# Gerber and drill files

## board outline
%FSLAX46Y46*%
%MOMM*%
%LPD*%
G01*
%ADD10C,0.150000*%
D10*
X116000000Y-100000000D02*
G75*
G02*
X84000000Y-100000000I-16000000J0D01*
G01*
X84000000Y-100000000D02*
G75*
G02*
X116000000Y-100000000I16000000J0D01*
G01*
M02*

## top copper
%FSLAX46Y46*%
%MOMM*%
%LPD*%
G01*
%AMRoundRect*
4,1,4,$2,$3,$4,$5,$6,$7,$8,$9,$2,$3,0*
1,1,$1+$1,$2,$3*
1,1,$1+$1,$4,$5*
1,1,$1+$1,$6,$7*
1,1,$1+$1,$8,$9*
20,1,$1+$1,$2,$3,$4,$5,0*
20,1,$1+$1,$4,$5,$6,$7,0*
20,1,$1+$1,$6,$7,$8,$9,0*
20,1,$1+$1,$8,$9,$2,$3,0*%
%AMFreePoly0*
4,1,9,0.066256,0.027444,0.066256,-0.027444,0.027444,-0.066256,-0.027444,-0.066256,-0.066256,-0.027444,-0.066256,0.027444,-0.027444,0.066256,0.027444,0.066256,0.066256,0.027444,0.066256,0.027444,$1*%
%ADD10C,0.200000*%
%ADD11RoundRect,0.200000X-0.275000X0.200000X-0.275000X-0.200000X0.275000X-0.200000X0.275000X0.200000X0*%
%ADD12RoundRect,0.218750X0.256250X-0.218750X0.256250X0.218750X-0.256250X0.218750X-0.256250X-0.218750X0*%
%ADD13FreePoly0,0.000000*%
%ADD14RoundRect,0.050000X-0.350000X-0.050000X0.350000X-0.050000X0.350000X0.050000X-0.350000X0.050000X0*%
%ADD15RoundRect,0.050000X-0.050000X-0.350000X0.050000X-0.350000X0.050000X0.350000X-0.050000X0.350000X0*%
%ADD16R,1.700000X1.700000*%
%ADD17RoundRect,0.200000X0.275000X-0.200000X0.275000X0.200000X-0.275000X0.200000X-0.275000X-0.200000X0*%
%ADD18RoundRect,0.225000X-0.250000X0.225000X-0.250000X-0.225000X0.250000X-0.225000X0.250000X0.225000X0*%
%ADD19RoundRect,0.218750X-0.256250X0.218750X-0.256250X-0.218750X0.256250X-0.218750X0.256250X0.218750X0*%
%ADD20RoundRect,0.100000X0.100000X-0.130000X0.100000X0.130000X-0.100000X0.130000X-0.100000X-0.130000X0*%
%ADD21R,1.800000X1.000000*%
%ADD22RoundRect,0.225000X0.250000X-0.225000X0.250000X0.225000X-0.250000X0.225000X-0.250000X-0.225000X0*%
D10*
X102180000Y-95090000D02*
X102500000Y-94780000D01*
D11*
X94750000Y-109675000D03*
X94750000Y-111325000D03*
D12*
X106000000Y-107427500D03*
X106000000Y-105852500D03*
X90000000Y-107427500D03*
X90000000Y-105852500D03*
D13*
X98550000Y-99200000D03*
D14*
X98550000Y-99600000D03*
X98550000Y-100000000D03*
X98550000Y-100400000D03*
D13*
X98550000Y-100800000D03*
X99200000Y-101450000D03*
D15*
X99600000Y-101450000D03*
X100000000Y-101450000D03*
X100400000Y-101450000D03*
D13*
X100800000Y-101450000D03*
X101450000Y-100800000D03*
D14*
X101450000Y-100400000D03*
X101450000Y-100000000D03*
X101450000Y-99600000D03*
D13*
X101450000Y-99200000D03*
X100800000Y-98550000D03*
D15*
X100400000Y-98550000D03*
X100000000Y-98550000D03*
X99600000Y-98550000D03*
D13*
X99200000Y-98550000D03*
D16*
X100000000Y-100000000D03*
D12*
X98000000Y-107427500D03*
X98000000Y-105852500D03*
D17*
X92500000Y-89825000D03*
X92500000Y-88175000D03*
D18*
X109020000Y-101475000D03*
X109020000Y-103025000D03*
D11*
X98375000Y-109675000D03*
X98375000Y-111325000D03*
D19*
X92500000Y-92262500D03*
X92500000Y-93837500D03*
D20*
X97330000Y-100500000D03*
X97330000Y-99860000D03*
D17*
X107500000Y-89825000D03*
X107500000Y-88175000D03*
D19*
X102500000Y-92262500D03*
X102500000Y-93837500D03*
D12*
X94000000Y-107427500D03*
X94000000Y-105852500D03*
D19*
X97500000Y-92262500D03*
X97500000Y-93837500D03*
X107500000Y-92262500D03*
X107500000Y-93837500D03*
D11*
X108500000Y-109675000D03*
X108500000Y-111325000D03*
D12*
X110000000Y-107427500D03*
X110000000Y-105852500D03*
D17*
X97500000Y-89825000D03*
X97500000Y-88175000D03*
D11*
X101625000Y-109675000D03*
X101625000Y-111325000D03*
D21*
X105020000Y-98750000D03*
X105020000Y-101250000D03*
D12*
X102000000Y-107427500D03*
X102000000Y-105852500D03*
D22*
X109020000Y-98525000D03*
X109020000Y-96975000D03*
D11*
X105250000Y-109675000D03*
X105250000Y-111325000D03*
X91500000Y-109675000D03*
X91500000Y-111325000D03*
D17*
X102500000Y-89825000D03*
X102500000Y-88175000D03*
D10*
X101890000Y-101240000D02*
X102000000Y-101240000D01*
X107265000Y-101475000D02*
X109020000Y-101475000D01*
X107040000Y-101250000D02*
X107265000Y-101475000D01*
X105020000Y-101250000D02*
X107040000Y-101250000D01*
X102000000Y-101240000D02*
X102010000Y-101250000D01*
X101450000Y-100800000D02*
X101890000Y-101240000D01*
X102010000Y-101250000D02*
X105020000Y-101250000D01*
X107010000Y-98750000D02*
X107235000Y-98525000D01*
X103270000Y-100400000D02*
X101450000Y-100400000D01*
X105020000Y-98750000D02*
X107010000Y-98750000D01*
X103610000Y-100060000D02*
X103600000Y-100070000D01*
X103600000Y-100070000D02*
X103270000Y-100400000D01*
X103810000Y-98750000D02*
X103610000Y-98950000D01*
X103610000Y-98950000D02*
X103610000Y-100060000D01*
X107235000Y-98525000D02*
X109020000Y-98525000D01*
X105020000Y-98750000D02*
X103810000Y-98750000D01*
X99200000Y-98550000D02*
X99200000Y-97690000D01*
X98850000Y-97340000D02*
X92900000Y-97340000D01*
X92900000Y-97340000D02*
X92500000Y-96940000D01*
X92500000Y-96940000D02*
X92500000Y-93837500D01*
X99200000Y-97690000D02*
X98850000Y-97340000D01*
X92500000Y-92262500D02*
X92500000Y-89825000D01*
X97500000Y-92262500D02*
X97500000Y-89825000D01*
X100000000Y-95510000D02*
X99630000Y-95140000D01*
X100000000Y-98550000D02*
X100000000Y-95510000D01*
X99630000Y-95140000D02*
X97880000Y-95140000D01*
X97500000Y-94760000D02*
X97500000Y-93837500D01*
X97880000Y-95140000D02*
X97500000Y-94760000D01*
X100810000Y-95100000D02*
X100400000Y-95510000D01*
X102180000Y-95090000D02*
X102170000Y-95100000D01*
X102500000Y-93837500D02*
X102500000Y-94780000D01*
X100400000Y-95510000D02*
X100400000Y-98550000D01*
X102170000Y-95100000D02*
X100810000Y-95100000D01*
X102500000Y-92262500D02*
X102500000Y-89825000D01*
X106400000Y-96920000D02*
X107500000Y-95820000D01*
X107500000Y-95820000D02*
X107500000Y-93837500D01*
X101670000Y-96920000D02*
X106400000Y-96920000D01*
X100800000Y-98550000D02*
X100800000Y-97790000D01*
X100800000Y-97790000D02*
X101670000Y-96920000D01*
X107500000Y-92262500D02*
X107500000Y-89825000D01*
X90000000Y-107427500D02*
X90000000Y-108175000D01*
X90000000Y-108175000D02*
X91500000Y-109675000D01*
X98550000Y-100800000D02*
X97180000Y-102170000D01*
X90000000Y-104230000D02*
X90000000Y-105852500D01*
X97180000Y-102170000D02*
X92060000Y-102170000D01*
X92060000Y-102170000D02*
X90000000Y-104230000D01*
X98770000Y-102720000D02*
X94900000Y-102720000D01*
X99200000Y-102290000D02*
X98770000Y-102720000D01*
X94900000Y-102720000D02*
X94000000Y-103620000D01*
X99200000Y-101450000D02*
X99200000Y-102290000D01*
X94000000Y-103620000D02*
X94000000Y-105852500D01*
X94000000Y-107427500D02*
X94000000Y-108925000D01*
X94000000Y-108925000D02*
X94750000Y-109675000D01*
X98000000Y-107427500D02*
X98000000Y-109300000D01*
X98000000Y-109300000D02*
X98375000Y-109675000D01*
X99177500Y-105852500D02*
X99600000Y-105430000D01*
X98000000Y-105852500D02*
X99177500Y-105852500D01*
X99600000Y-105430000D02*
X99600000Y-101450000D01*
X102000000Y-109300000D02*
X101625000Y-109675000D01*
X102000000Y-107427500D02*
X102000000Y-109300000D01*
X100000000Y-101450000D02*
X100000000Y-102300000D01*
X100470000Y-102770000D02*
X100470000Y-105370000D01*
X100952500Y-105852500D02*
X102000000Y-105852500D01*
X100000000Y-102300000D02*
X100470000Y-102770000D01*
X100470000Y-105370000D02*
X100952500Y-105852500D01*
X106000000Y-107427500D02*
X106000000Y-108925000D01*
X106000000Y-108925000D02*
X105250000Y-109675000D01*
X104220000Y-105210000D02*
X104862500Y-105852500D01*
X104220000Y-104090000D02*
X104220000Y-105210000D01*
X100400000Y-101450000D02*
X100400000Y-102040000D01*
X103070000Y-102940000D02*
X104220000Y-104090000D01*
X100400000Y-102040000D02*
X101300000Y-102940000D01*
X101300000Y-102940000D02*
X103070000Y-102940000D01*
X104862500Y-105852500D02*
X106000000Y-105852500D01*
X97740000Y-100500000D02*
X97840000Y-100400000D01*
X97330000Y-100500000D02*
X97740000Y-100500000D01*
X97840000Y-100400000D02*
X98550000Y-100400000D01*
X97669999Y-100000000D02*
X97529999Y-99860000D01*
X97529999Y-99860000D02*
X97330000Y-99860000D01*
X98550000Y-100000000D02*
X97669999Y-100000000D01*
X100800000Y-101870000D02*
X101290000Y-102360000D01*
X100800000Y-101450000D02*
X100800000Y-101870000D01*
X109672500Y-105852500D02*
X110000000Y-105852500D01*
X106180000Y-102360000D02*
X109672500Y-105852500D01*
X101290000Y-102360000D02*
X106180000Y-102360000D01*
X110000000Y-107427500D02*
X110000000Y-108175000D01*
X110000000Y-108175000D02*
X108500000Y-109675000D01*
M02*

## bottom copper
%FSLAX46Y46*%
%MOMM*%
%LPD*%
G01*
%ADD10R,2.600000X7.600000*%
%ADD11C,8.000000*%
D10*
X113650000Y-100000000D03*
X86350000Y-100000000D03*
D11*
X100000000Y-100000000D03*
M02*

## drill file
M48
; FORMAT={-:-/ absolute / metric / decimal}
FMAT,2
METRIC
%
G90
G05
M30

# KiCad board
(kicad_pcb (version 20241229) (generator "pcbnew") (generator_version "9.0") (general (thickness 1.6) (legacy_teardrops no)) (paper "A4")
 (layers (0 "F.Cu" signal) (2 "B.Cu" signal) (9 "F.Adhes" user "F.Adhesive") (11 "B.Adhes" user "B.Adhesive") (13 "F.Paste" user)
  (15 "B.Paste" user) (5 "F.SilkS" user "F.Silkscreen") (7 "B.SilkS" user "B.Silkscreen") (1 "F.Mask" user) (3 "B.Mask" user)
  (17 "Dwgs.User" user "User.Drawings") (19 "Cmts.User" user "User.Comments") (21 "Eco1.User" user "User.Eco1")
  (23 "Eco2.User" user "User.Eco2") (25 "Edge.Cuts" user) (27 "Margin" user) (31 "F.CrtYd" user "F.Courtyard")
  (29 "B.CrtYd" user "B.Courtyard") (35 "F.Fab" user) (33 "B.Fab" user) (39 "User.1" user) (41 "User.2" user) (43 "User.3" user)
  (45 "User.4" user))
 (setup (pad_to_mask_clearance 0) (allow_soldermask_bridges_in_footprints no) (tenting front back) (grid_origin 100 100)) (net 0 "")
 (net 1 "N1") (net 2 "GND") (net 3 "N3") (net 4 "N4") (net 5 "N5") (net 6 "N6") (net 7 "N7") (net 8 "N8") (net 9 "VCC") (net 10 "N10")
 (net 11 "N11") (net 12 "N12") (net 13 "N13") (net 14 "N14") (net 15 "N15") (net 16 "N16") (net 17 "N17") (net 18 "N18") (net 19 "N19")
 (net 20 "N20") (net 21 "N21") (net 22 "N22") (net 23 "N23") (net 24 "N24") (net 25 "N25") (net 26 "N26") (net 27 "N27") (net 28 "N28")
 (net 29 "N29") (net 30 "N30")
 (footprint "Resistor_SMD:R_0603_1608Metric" (layer "F.Cu") (at 94.75 110.5 -90)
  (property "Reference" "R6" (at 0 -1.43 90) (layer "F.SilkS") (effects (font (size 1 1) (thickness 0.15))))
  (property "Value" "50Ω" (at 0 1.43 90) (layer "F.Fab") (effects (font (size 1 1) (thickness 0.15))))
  (pad "1" smd roundrect (at -0.825 0 270) (size 0.8 0.95) (layers "F.Cu" "F.Mask" "F.Paste") (roundrect_rratio 0.25) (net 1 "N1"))
  (pad "2" smd roundrect (at 0.825 0 270) (size 0.8 0.95) (layers "F.Cu" "F.Mask" "F.Paste") (roundrect_rratio 0.25) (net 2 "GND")))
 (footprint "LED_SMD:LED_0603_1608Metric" (layer "F.Cu") (at 106 106.64 90)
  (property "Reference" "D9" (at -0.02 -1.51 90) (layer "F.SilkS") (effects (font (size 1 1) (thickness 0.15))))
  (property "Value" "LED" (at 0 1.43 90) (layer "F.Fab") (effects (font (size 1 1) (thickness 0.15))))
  (pad "1" smd roundrect (at -0.7875 0 90) (size 0.875 0.95) (layers "F.Cu" "F.Mask" "F.Paste") (roundrect_rratio 0.25) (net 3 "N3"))
  (pad "2" smd roundrect (at 0.7875 0 90) (size 0.875 0.95) (layers "F.Cu" "F.Mask" "F.Paste") (roundrect_rratio 0.25) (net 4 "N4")))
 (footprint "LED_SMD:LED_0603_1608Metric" (layer "F.Cu") (at 90 106.64 90)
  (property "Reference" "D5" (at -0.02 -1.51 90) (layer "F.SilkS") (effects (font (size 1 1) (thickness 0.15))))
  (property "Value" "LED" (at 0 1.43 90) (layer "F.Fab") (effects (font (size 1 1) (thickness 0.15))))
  (pad "1" smd roundrect (at -0.7875 0 90) (size 0.875 0.95) (layers "F.Cu" "F.Mask" "F.Paste") (roundrect_rratio 0.25) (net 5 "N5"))
  (pad "2" smd roundrect (at 0.7875 0 90) (size 0.875 0.95) (layers "F.Cu" "F.Mask" "F.Paste") (roundrect_rratio 0.25) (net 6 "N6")))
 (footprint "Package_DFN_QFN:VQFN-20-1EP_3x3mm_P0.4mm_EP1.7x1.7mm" (layer "F.Cu") (at 100 100)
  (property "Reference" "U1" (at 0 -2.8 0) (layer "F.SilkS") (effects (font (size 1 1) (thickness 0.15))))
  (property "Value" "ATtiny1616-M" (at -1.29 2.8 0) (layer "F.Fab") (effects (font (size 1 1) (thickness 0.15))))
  (pad "" smd roundrect (at -0.425 -0.425) (size 0.69 0.69) (layers "F.Paste") (roundrect_rratio 0.25))
  (pad "" smd roundrect (at -0.425 0.425) (size 0.69 0.69) (layers "F.Paste") (roundrect_rratio 0.25))
  (pad "" smd roundrect (at 0.425 -0.425) (size 0.69 0.69) (layers "F.Paste") (roundrect_rratio 0.25))
  (pad "" smd roundrect (at 0.425 0.425) (size 0.69 0.69) (layers "F.Paste") (roundrect_rratio 0.25))
  (pad "1" smd custom (at -1.45 -0.8) (size 0.143431 0.143431) (layers "F.Cu" "F.Mask" "F.Paste") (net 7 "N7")
   (options (clearance outline) (anchor circle)) (primitives))
  (pad "2" smd roundrect (at -1.45 -0.4) (size 0.8 0.2) (layers "F.Cu" "F.Mask" "F.Paste") (roundrect_rratio 0.25) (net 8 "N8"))
  (pad "3" smd roundrect (at -1.45 0) (size 0.8 0.2) (layers "F.Cu" "F.Mask" "F.Paste") (roundrect_rratio 0.25) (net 2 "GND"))
  (pad "4" smd roundrect (at -1.45 0.4) (size 0.8 0.2) (layers "F.Cu" "F.Mask" "F.Paste") (roundrect_rratio 0.25) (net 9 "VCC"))
  (pad "5" smd custom (at -1.45 0.8) (size 0.143431 0.143431) (layers "F.Cu" "F.Mask" "F.Paste") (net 6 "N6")
   (options (clearance outline) (anchor circle)) (primitives))
  (pad "6" smd custom (at -0.8 1.45) (size 0.143431 0.143431) (layers "F.Cu" "F.Mask" "F.Paste") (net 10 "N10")
   (options (clearance outline) (anchor circle)) (primitives))
  (pad "7" smd roundrect (at -0.4 1.45) (size 0.2 0.8) (layers "F.Cu" "F.Mask" "F.Paste") (roundrect_rratio 0.25) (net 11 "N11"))
  (pad "8" smd roundrect (at 0 1.45) (size 0.2 0.8) (layers "F.Cu" "F.Mask" "F.Paste") (roundrect_rratio 0.25) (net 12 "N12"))
  (pad "9" smd roundrect (at 0.4 1.45) (size 0.2 0.8) (layers "F.Cu" "F.Mask" "F.Paste") (roundrect_rratio 0.25) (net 4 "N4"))
  (pad "10" smd custom (at 0.8 1.45) (size 0.143431 0.143431) (layers "F.Cu" "F.Mask" "F.Paste") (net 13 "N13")
   (options (clearance outline) (anchor circle)) (primitives))
  (pad "11" smd custom (at 1.45 0.8) (size 0.143431 0.143431) (layers "F.Cu" "F.Mask" "F.Paste") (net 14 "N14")
   (options (clearance outline) (anchor circle)) (primitives))
  (pad "12" smd roundrect (at 1.45 0.4) (size 0.8 0.2) (layers "F.Cu" "F.Mask" "F.Paste") (roundrect_rratio 0.25) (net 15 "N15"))
  (pad "13" smd roundrect (at 1.45 0) (size 0.8 0.2) (layers "F.Cu" "F.Mask" "F.Paste") (roundrect_rratio 0.25) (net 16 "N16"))
  (pad "14" smd roundrect (at 1.45 -0.4) (size 0.8 0.2) (layers "F.Cu" "F.Mask" "F.Paste") (roundrect_rratio 0.25) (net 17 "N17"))
  (pad "15" smd custom (at 1.45 -0.8) (size 0.143431 0.143431) (layers "F.Cu" "F.Mask" "F.Paste") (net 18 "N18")
   (options (clearance outline) (anchor circle)) (primitives))
  (pad "16" smd custom (at 0.8 -1.45) (size 0.143431 0.143431) (layers "F.Cu" "F.Mask" "F.Paste") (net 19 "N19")
   (options (clearance outline) (anchor circle)) (primitives))
  (pad "17" smd roundrect (at 0.4 -1.45) (size 0.2 0.8) (layers "F.Cu" "F.Mask" "F.Paste") (roundrect_rratio 0.25) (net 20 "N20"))
  (pad "18" smd roundrect (at 0 -1.45) (size 0.2 0.8) (layers "F.Cu" "F.Mask" "F.Paste") (roundrect_rratio 0.25) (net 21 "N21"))
  (pad "19" smd roundrect (at -0.4 -1.45) (size 0.2 0.8) (layers "F.Cu" "F.Mask" "F.Paste") (roundrect_rratio 0.25) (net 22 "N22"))
  (pad "20" smd custom (at -0.8 -1.45) (size 0.143431 0.143431) (layers "F.Cu" "F.Mask" "F.Paste") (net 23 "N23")
   (options (clearance outline) (anchor circle)) (primitives))
  (pad "21" smd rect (at 0 0) (size 1.7 1.7) (layers "F.Cu" "F.Mask") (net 2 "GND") (zone_connect 2)))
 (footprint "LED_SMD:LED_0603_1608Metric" (layer "F.Cu") (at 98 106.64 90)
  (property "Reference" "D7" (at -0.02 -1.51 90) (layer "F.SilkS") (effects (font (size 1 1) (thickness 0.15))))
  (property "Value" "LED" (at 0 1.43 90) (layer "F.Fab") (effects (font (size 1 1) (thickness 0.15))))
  (pad "1" smd roundrect (at -0.7875 0 90) (size 0.875 0.95) (layers "F.Cu" "F.Mask" "F.Paste") (roundrect_rratio 0.25) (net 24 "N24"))
  (pad "2" smd roundrect (at 0.7875 0 90) (size 0.875 0.95) (layers "F.Cu" "F.Mask" "F.Paste") (roundrect_rratio 0.25) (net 11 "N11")))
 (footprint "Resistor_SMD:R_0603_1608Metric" (layer "F.Cu") (at 92.5 89 90)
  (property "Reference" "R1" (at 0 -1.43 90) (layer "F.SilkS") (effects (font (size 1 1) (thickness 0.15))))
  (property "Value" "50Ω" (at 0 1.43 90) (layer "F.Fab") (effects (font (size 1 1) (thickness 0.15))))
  (pad "1" smd roundrect (at -0.825 0 90) (size 0.8 0.95) (layers "F.Cu" "F.Mask" "F.Paste") (roundrect_rratio 0.25) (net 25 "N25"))
  (pad "2" smd roundrect (at 0.825 0 90) (size 0.8 0.95) (layers "F.Cu" "F.Mask" "F.Paste") (roundrect_rratio 0.25) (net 2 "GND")))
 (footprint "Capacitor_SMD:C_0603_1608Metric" (layer "F.Cu") (at 109.02 102.25 -90)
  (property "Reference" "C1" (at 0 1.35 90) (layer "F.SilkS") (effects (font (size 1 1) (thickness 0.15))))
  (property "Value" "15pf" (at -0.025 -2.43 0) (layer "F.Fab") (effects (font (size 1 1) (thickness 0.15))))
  (pad "1" smd roundrect (at -0.775 0 270) (size 0.9 0.95) (layers "F.Cu" "F.Mask" "F.Paste") (roundrect_rratio 0.25) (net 14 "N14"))
  (pad "2" smd roundrect (at 0.775 0 270) (size 0.9 0.95) (layers "F.Cu" "F.Mask" "F.Paste") (roundrect_rratio 0.25) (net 2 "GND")))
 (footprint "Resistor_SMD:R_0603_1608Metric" (layer "F.Cu") (at 98.375 110.5 -90)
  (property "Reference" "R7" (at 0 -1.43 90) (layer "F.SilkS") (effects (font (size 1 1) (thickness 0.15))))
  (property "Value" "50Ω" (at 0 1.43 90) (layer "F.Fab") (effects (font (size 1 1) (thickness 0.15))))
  (pad "1" smd roundrect (at -0.825 0 270) (size 0.8 0.95) (layers "F.Cu" "F.Mask" "F.Paste") (roundrect_rratio 0.25) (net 24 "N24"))
  (pad "2" smd roundrect (at 0.825 0 270) (size 0.8 0.95) (layers "F.Cu" "F.Mask" "F.Paste") (roundrect_rratio 0.25) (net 2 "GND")))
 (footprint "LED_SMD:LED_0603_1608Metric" (layer "F.Cu") (at 92.5 93.05 -90)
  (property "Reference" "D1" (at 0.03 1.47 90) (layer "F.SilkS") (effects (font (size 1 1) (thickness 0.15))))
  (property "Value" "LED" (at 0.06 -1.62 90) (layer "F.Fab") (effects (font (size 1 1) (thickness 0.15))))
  (pad "1" smd roundrect (at -0.7875 0 270) (size 0.875 0.95) (layers "F.Cu" "F.Mask" "F.Paste") (roundrect_rratio 0.25) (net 25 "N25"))
  (pad "2" smd roundrect (at 0.7875 0 270) (size 0.875 0.95) (layers "F.Cu" "F.Mask" "F.Paste") (roundrect_rratio 0.25) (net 23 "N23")))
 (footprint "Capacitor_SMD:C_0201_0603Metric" (layer "F.Cu") (at 97.33 100.18 90)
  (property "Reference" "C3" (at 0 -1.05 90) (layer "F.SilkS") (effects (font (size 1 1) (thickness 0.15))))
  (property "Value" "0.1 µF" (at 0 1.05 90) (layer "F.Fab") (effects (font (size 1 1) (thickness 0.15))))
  (pad "" smd roundrect (at -0.345 0 90) (size 0.318 0.36) (layers "F.Paste") (roundrect_rratio 0.25))
  (pad "" smd roundrect (at 0.345 0 90) (size 0.318 0.36) (layers "F.Paste") (roundrect_rratio 0.25))
  (pad "1" smd roundrect (at -0.32 0 90) (size 0.46 0.4) (layers "F.Cu" "F.Mask") (roundrect_rratio 0.25) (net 9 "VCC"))
  (pad "2" smd roundrect (at 0.32 0 90) (size 0.46 0.4) (layers "F.Cu" "F.Mask") (roundrect_rratio 0.25) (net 2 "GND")))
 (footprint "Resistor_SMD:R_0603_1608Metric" (layer "F.Cu") (at 107.5 89 90)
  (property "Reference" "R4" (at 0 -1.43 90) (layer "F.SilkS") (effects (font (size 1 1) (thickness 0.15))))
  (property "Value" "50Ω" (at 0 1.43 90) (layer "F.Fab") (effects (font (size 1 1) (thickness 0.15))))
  (pad "1" smd roundrect (at -0.825 0 90) (size 0.8 0.95) (layers "F.Cu" "F.Mask" "F.Paste") (roundrect_rratio 0.25) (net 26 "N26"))
  (pad "2" smd roundrect (at 0.825 0 90) (size 0.8 0.95) (layers "F.Cu" "F.Mask" "F.Paste") (roundrect_rratio 0.25) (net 2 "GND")))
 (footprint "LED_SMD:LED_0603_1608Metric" (layer "F.Cu") (at 102.5 93.05 -90)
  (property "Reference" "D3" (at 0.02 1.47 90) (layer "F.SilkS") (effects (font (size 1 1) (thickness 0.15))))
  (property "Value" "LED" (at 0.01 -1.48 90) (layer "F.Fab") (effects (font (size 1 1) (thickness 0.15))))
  (pad "1" smd roundrect (at -0.7875 0 270) (size 0.875 0.95) (layers "F.Cu" "F.Mask" "F.Paste") (roundrect_rratio 0.25) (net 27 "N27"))
  (pad "2" smd roundrect (at 0.7875 0 270) (size 0.875 0.95) (layers "F.Cu" "F.Mask" "F.Paste") (roundrect_rratio 0.25) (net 20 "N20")))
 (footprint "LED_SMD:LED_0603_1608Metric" (layer "F.Cu") (at 94 106.64 90)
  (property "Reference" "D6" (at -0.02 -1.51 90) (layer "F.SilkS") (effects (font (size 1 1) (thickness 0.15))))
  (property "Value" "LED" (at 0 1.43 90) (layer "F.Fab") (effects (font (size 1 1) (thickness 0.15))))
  (pad "1" smd roundrect (at -0.7875 0 90) (size 0.875 0.95) (layers "F.Cu" "F.Mask" "F.Paste") (roundrect_rratio 0.25) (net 1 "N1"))
  (pad "2" smd roundrect (at 0.7875 0 90) (size 0.875 0.95) (layers "F.Cu" "F.Mask" "F.Paste") (roundrect_rratio 0.25) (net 10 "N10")))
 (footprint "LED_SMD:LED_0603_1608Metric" (layer "F.Cu") (at 97.5 93.05 -90)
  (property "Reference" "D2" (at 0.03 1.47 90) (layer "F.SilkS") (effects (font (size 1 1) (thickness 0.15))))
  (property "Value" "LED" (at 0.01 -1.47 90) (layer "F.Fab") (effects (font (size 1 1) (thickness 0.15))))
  (pad "1" smd roundrect (at -0.7875 0 270) (size 0.875 0.95) (layers "F.Cu" "F.Mask" "F.Paste") (roundrect_rratio 0.25) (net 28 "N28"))
  (pad "2" smd roundrect (at 0.7875 0 270) (size 0.875 0.95) (layers "F.Cu" "F.Mask" "F.Paste") (roundrect_rratio 0.25) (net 21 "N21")))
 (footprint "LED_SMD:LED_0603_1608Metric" (layer "F.Cu") (at 107.5 93.05 -90)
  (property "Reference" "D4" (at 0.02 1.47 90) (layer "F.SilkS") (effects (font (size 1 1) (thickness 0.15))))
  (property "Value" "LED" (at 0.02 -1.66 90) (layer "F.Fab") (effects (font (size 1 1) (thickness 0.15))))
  (pad "1" smd roundrect (at -0.7875 0 270) (size 0.875 0.95) (layers "F.Cu" "F.Mask" "F.Paste") (roundrect_rratio 0.25) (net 26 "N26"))
  (pad "2" smd roundrect (at 0.7875 0 270) (size 0.875 0.95) (layers "F.Cu" "F.Mask" "F.Paste") (roundrect_rratio 0.25) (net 19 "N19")))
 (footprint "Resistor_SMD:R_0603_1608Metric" (layer "F.Cu") (at 108.5 110.5 -90)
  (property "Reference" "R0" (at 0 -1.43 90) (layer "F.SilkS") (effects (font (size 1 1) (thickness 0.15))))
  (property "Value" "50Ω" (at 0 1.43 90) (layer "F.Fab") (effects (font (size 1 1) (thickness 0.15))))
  (pad "1" smd roundrect (at -0.825 0 270) (size 0.8 0.95) (layers "F.Cu" "F.Mask" "F.Paste") (roundrect_rratio 0.25) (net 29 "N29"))
  (pad "2" smd roundrect (at 0.825 0 270) (size 0.8 0.95) (layers "F.Cu" "F.Mask" "F.Paste") (roundrect_rratio 0.25) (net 2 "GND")))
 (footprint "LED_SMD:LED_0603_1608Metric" (layer "F.Cu") (at 110 106.64 90)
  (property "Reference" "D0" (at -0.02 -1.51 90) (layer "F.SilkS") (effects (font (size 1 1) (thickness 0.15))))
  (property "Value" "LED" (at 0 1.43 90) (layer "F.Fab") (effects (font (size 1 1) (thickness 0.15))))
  (pad "1" smd roundrect (at -0.7875 0 90) (size 0.875 0.95) (layers "F.Cu" "F.Mask" "F.Paste") (roundrect_rratio 0.25) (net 29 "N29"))
  (pad "2" smd roundrect (at 0.7875 0 90) (size 0.875 0.95) (layers "F.Cu" "F.Mask" "F.Paste") (roundrect_rratio 0.25) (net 13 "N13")))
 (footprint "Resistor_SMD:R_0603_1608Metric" (layer "F.Cu") (at 97.5 89 90)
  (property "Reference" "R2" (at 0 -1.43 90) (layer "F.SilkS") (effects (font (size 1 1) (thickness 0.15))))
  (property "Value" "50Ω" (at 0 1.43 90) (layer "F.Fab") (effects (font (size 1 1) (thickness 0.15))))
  (pad "1" smd roundrect (at -0.825 0 90) (size 0.8 0.95) (layers "F.Cu" "F.Mask" "F.Paste") (roundrect_rratio 0.25) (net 28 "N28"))
  (pad "2" smd roundrect (at 0.825 0 90) (size 0.8 0.95) (layers "F.Cu" "F.Mask" "F.Paste") (roundrect_rratio 0.25) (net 2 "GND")))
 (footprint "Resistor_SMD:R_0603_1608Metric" (layer "F.Cu") (at 101.625 110.5 -90)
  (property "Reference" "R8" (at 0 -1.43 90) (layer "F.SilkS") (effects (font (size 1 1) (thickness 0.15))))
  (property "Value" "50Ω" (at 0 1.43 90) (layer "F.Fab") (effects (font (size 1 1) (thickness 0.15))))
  (pad "1" smd roundrect (at -0.825 0 270) (size 0.8 0.95) (layers "F.Cu" "F.Mask" "F.Paste") (roundrect_rratio 0.25) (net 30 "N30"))
  (pad "2" smd roundrect (at 0.825 0 270) (size 0.8 0.95) (layers "F.Cu" "F.Mask" "F.Paste") (roundrect_rratio 0.25) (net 2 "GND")))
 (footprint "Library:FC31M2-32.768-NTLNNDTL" (layer "F.Cu") (at 105.02 100)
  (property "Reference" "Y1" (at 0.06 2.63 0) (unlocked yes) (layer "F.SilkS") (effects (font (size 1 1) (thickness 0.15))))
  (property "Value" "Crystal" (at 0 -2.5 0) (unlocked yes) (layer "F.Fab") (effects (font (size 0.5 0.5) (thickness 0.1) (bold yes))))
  (pad "1" smd rect (at 0 -1.25 180) (size 1.8 1) (layers "F.Cu" "F.Mask" "F.Paste") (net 15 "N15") (thermal_bridge_angle 45))
  (pad "2" smd rect (at 0 1.25 180) (size 1.8 1) (layers "F.Cu" "F.Mask" "F.Paste") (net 14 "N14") (thermal_bridge_angle 45)))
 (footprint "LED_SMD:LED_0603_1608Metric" (layer "F.Cu") (at 102 106.64 90)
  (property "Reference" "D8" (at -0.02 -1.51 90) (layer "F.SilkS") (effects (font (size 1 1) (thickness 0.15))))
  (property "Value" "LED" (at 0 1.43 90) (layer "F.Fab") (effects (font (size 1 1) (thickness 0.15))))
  (pad "1" smd roundrect (at -0.7875 0 90) (size 0.875 0.95) (layers "F.Cu" "F.Mask" "F.Paste") (roundrect_rratio 0.25) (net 30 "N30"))
  (pad "2" smd roundrect (at 0.7875 0 90) (size 0.875 0.95) (layers "F.Cu" "F.Mask" "F.Paste") (roundrect_rratio 0.25) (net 12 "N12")))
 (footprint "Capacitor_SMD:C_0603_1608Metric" (layer "F.Cu") (at 109.02 97.75 90)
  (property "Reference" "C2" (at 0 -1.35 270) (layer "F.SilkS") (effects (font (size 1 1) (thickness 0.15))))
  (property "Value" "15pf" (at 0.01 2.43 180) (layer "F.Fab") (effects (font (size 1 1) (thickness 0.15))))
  (pad "1" smd roundrect (at -0.775 0 90) (size 0.9 0.95) (layers "F.Cu" "F.Mask" "F.Paste") (roundrect_rratio 0.25) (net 15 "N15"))
  (pad "2" smd roundrect (at 0.775 0 90) (size 0.9 0.95) (layers "F.Cu" "F.Mask" "F.Paste") (roundrect_rratio 0.25) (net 2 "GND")))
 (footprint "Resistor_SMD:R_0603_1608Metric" (layer "F.Cu") (at 105.25 110.5 -90)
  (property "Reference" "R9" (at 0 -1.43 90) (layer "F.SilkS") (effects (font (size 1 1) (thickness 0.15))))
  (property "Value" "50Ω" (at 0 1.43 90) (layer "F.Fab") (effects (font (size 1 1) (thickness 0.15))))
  (pad "1" smd roundrect (at -0.825 0 270) (size 0.8 0.95) (layers "F.Cu" "F.Mask" "F.Paste") (roundrect_rratio 0.25) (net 3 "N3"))
  (pad "2" smd roundrect (at 0.825 0 270) (size 0.8 0.95) (layers "F.Cu" "F.Mask" "F.Paste") (roundrect_rratio 0.25) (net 2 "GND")))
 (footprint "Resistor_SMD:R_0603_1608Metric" (layer "F.Cu") (at 91.5 110.5 -90)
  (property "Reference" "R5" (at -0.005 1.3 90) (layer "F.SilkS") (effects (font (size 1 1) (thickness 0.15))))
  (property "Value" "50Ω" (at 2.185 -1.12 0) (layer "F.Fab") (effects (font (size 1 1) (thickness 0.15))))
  (pad "1" smd roundrect (at -0.825 0 270) (size 0.8 0.95) (layers "F.Cu" "F.Mask" "F.Paste") (roundrect_rratio 0.25) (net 5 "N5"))
  (pad "2" smd roundrect (at 0.825 0 270) (size 0.8 0.95) (layers "F.Cu" "F.Mask" "F.Paste") (roundrect_rratio 0.25) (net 2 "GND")))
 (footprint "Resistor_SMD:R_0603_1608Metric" (layer "F.Cu") (at 102.5 89 90)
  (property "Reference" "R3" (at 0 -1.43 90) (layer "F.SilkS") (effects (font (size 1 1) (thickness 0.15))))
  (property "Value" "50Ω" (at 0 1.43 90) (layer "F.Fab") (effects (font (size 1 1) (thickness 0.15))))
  (pad "1" smd roundrect (at -0.825 0 90) (size 0.8 0.95) (layers "F.Cu" "F.Mask" "F.Paste") (roundrect_rratio 0.25) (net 27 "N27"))
  (pad "2" smd roundrect (at 0.825 0 90) (size 0.8 0.95) (layers "F.Cu" "F.Mask" "F.Paste") (roundrect_rratio 0.25) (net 2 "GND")))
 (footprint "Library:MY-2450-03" (layer "B.Cu") (at 100 100 180)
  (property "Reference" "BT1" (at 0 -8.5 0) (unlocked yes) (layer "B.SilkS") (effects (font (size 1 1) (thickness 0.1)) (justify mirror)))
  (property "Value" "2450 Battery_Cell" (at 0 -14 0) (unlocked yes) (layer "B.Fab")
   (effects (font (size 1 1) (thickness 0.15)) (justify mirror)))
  (pad "1" smd rect (at -13.65 0 180) (size 2.6 7.6) (layers "B.Cu" "B.Mask" "B.Paste") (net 9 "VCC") (thermal_bridge_angle 45))
  (pad "1" smd rect (at 13.65 0 180) (size 2.6 7.6) (layers "B.Cu" "B.Mask" "B.Paste") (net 9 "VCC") (thermal_bridge_angle 45))
  (pad "2" smd circle (at 0 0 180) (size 8 8) (layers "B.Cu" "B.Mask" "B.Paste") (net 2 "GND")))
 (gr_line (start 102.18 95.09) (end 102.5 94.78) (stroke (width 0.2) (type default)) (layer "F.Cu") (net 20))
 (gr_circle (center 100 100) (end 116 100) (stroke (width 0.15) (type solid)) (fill no) (layer "Edge.Cuts"))
 (segment (start 101.89 101.24) (end 102 101.24) (width 0.2) (layer "F.Cu") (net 14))
 (segment (start 107.265 101.475) (end 109.02 101.475) (width 0.2) (layer "F.Cu") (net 14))
 (segment (start 107.04 101.25) (end 107.265 101.475) (width 0.2) (layer "F.Cu") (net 14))
 (segment (start 105.02 101.25) (end 107.04 101.25) (width 0.2) (layer "F.Cu") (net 14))
 (segment (start 102 101.24) (end 102.01 101.25) (width 0.2) (layer "F.Cu") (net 14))
 (segment (start 101.45 100.8) (end 101.89 101.24) (width 0.2) (layer "F.Cu") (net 14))
 (segment (start 102.01 101.25) (end 105.02 101.25) (width 0.2) (layer "F.Cu") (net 14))
 (segment (start 107.01 98.75) (end 107.235 98.525) (width 0.2) (layer "F.Cu") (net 15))
 (segment (start 103.27 100.4) (end 101.45 100.4) (width 0.2) (layer "F.Cu") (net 15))
 (segment (start 105.02 98.75) (end 107.01 98.75) (width 0.2) (layer "F.Cu") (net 15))
 (segment (start 103.61 100.06) (end 103.6 100.07) (width 0.2) (layer "F.Cu") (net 15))
 (segment (start 103.6 100.07) (end 103.27 100.4) (width 0.2) (layer "F.Cu") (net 15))
 (segment (start 103.81 98.75) (end 103.61 98.95) (width 0.2) (layer "F.Cu") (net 15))
 (segment (start 103.61 98.95) (end 103.61 100.06) (width 0.2) (layer "F.Cu") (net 15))
 (segment (start 107.235 98.525) (end 109.02 98.525) (width 0.2) (layer "F.Cu") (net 15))
 (segment (start 105.02 98.75) (end 103.81 98.75) (width 0.2) (layer "F.Cu") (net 15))
 (segment (start 99.2 98.55) (end 99.2 97.69) (width 0.2) (layer "F.Cu") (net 23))
 (segment (start 98.85 97.34) (end 92.9 97.34) (width 0.2) (layer "F.Cu") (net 23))
 (segment (start 92.9 97.34) (end 92.5 96.94) (width 0.2) (layer "F.Cu") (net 23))
 (segment (start 92.5 96.94) (end 92.5 93.8375) (width 0.2) (layer "F.Cu") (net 23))
 (segment (start 99.2 97.69) (end 98.85 97.34) (width 0.2) (layer "F.Cu") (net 23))
 (segment (start 92.5 92.2625) (end 92.5 89.825) (width 0.2) (layer "F.Cu") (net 25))
 (segment (start 97.5 92.2625) (end 97.5 89.825) (width 0.2) (layer "F.Cu") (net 28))
 (segment (start 100 95.51) (end 99.63 95.14) (width 0.2) (layer "F.Cu") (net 21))
 (segment (start 100 98.55) (end 100 95.51) (width 0.2) (layer "F.Cu") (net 21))
 (segment (start 99.63 95.14) (end 97.88 95.14) (width 0.2) (layer "F.Cu") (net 21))
 (segment (start 97.5 94.76) (end 97.5 93.8375) (width 0.2) (layer "F.Cu") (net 21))
 (segment (start 97.88 95.14) (end 97.5 94.76) (width 0.2) (layer "F.Cu") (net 21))
 (segment (start 100.81 95.1) (end 100.4 95.51) (width 0.2) (layer "F.Cu") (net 20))
 (segment (start 102.18 95.09) (end 102.17 95.1) (width 0.2) (layer "F.Cu") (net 20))
 (segment (start 102.5 93.8375) (end 102.5 94.78) (width 0.2) (layer "F.Cu") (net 20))
 (segment (start 100.4 95.51) (end 100.4 98.55) (width 0.2) (layer "F.Cu") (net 20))
 (segment (start 102.17 95.1) (end 100.81 95.1) (width 0.2) (layer "F.Cu") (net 20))
 (segment (start 102.5 92.2625) (end 102.5 89.825) (width 0.2) (layer "F.Cu") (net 27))
 (segment (start 106.4 96.92) (end 107.5 95.82) (width 0.2) (layer "F.Cu") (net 19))
 (segment (start 107.5 95.82) (end 107.5 93.8375) (width 0.2) (layer "F.Cu") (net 19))
 (segment (start 101.67 96.92) (end 106.4 96.92) (width 0.2) (layer "F.Cu") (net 19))
 (segment (start 100.8 98.55) (end 100.8 97.79) (width 0.2) (layer "F.Cu") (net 19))
 (segment (start 100.8 97.79) (end 101.67 96.92) (width 0.2) (layer "F.Cu") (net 19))
 (segment (start 107.5 92.2625) (end 107.5 89.825) (width 0.2) (layer "F.Cu") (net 26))
 (segment (start 90 107.4275) (end 90 108.175) (width 0.2) (layer "F.Cu") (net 5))
 (segment (start 90 108.175) (end 91.5 109.675) (width 0.2) (layer "F.Cu") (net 5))
 (segment (start 98.55 100.8) (end 97.18 102.17) (width 0.2) (layer "F.Cu") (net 6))
 (segment (start 90 104.23) (end 90 105.8525) (width 0.2) (layer "F.Cu") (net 6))
 (segment (start 97.18 102.17) (end 92.06 102.17) (width 0.2) (layer "F.Cu") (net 6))
 (segment (start 92.06 102.17) (end 90 104.23) (width 0.2) (layer "F.Cu") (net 6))
 (segment (start 98.77 102.72) (end 94.9 102.72) (width 0.2) (layer "F.Cu") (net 10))
 (segment (start 99.2 102.29) (end 98.77 102.72) (width 0.2) (layer "F.Cu") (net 10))
 (segment (start 94.9 102.72) (end 94 103.62) (width 0.2) (layer "F.Cu") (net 10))
 (segment (start 99.2 101.45) (end 99.2 102.29) (width 0.2) (layer "F.Cu") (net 10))
 (segment (start 94 103.62) (end 94 105.8525) (width 0.2) (layer "F.Cu") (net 10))
 (segment (start 94 107.4275) (end 94 108.925) (width 0.2) (layer "F.Cu") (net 1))
 (segment (start 94 108.925) (end 94.75 109.675) (width 0.2) (layer "F.Cu") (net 1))
 (segment (start 98 107.4275) (end 98 109.3) (width 0.2) (layer "F.Cu") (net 24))
 (segment (start 98 109.3) (end 98.375 109.675) (width 0.2) (layer "F.Cu") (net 24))
 (segment (start 99.1775 105.8525) (end 99.6 105.43) (width 0.2) (layer "F.Cu") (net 11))
 (segment (start 98 105.8525) (end 99.1775 105.8525) (width 0.2) (layer "F.Cu") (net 11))
 (segment (start 99.6 105.43) (end 99.6 101.45) (width 0.2) (layer "F.Cu") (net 11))
 (segment (start 102 109.3) (end 101.625 109.675) (width 0.2) (layer "F.Cu") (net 30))
 (segment (start 102 107.4275) (end 102 109.3) (width 0.2) (layer "F.Cu") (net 30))
 (segment (start 100 101.45) (end 100 102.3) (width 0.2) (layer "F.Cu") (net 12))
 (segment (start 100.47 102.77) (end 100.47 105.37) (width 0.2) (layer "F.Cu") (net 12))
 (segment (start 100.9525 105.8525) (end 102 105.8525) (width 0.2) (layer "F.Cu") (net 12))
 (segment (start 100 102.3) (end 100.47 102.77) (width 0.2) (layer "F.Cu") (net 12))
 (segment (start 100.47 105.37) (end 100.9525 105.8525) (width 0.2) (layer "F.Cu") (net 12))
 (segment (start 106 107.4275) (end 106 108.925) (width 0.2) (layer "F.Cu") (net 3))
 (segment (start 106 108.925) (end 105.25 109.675) (width 0.2) (layer "F.Cu") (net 3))
 (segment (start 104.22 105.21) (end 104.8625 105.8525) (width 0.2) (layer "F.Cu") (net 4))
 (segment (start 104.22 104.09) (end 104.22 105.21) (width 0.2) (layer "F.Cu") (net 4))
 (segment (start 100.4 101.45) (end 100.4 102.04) (width 0.2) (layer "F.Cu") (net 4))
 (segment (start 103.07 102.94) (end 104.22 104.09) (width 0.2) (layer "F.Cu") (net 4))
 (segment (start 100.4 102.04) (end 101.3 102.94) (width 0.2) (layer "F.Cu") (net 4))
 (segment (start 101.3 102.94) (end 103.07 102.94) (width 0.2) (layer "F.Cu") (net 4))
 (segment (start 104.8625 105.8525) (end 106 105.8525) (width 0.2) (layer "F.Cu") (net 4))
 (segment (start 97.74 100.5) (end 97.84 100.4) (width 0.2) (layer "F.Cu") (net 9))
 (segment (start 97.33 100.5) (end 97.74 100.5) (width 0.2) (layer "F.Cu") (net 9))
 (segment (start 97.84 100.4) (end 98.55 100.4) (width 0.2) (layer "F.Cu") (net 9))
 (segment (start 97.669999 100) (end 97.529999 99.86) (width 0.2) (layer "F.Cu") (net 2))
 (segment (start 97.529999 99.86) (end 97.33 99.86) (width 0.2) (layer "F.Cu") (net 2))
 (segment (start 98.55 100) (end 97.669999 100) (width 0.2) (layer "F.Cu") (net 2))
 (segment (start 100.8 101.87) (end 101.29 102.36) (width 0.2) (layer "F.Cu") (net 13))
 (segment (start 100.8 101.45) (end 100.8 101.87) (width 0.2) (layer "F.Cu") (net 13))
 (segment (start 109.6725 105.8525) (end 110 105.8525) (width 0.2) (layer "F.Cu") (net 13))
 (segment (start 106.18 102.36) (end 109.6725 105.8525) (width 0.2) (layer "F.Cu") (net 13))
 (segment (start 101.29 102.36) (end 106.18 102.36) (width 0.2) (layer "F.Cu") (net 13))
 (segment (start 110 107.4275) (end 110 108.175) (width 0.2) (layer "F.Cu") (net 29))
 (segment (start 110 108.175) (end 108.5 109.675) (width 0.2) (layer "F.Cu") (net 29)))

